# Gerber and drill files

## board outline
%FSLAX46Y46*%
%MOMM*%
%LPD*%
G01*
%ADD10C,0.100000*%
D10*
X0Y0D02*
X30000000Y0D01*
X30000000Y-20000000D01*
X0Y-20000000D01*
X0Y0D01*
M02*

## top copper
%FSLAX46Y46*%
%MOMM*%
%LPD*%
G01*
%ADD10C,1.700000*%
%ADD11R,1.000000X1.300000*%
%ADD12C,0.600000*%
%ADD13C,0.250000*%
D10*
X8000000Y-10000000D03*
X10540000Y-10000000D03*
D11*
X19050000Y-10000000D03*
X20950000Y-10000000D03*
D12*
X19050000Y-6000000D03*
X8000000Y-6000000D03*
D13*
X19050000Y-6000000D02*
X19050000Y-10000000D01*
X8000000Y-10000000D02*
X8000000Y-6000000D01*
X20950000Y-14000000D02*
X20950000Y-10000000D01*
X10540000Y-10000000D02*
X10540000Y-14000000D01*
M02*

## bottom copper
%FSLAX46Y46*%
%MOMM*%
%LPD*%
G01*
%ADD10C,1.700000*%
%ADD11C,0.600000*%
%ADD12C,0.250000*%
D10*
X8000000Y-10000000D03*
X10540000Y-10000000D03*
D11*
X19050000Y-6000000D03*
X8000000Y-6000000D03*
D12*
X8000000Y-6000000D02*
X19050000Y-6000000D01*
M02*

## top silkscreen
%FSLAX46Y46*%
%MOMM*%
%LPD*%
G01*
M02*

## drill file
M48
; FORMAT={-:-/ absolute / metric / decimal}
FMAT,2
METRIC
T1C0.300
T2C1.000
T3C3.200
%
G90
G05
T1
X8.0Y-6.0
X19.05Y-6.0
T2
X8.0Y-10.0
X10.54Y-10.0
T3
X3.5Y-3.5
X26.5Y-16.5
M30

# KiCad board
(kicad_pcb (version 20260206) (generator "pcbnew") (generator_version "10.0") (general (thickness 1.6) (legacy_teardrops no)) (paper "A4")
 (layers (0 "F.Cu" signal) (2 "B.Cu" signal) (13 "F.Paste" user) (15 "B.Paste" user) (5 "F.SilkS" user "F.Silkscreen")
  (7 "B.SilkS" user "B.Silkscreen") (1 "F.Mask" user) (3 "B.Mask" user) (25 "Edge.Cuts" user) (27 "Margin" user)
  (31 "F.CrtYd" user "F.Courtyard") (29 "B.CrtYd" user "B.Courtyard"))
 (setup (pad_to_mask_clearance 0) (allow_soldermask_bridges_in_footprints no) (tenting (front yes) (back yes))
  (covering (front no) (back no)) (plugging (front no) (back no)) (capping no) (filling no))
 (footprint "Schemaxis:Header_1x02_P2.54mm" (layer "F.Cu") (at 8 10 90)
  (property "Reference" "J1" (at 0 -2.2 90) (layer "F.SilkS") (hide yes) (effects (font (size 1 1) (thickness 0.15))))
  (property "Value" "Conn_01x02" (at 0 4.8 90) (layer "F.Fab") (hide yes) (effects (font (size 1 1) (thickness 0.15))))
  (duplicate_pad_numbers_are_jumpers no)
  (pad "1" thru_hole circle (at 0 0 90) (size 1.7 1.7) (drill 1) (layers "*.Cu" "*.Mask") (remove_unused_layers no) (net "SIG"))
  (pad "2" thru_hole circle (at 0 2.54 90) (size 1.7 1.7) (drill 1) (layers "*.Cu" "*.Mask") (remove_unused_layers no) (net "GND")))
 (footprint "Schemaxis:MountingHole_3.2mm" (layer "F.Cu") (at 3.5 3.5)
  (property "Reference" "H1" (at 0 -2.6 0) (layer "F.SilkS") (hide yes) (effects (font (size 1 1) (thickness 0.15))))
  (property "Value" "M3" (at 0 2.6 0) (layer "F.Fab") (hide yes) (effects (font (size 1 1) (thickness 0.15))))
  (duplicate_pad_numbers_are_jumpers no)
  (pad "" np_thru_hole circle (at 0 0) (size 3.2 3.2) (drill 3.2) (layers "*.Cu" "*.Mask")))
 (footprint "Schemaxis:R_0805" (layer "F.Cu") (at 20 10)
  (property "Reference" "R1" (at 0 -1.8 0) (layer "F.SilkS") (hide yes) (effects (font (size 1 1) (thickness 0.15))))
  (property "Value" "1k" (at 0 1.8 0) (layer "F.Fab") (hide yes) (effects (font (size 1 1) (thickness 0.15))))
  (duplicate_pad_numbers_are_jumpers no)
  (pad "1" smd rect (at -0.95 0) (size 1 1.3) (layers "F.Cu" "F.Mask" "F.Paste") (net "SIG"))
  (pad "2" smd rect (at 0.95 0) (size 1 1.3) (layers "F.Cu" "F.Mask" "F.Paste") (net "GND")))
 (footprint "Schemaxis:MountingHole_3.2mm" (layer "F.Cu") (at 26.5 16.5)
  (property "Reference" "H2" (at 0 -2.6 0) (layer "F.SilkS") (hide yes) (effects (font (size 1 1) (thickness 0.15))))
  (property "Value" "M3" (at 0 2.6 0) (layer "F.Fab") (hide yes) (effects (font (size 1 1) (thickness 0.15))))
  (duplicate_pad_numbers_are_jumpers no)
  (pad "" np_thru_hole circle (at 0 0) (size 3.2 3.2) (drill 3.2) (layers "*.Cu" "*.Mask")))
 (gr_rect (start 0 0) (end 30 20) (stroke (width 0.1) (type default)) (fill no) (layer "Edge.Cuts"))
 (segment (start 19.05 6) (end 19.05 10) (width 0.25) (layer "F.Cu") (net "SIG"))
 (segment (start 8 10) (end 8 6) (width 0.25) (layer "F.Cu") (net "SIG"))
 (via (at 19.05 6) (size 0.6) (drill 0.3) (layers "F.Cu" "B.Cu") (capping no) (covering (front no) (back no))
  (plugging (front no) (back no)) (filling no) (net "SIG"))
 (via (at 8 6) (size 0.6) (drill 0.3) (layers "F.Cu" "B.Cu") (capping no) (covering (front no) (back no)) (plugging (front no) (back no))
  (filling no) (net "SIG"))
 (segment (start 8 6) (end 19.05 6) (width 0.25) (layer "B.Cu") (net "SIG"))
 (segment (start 20.95 14) (end 20.95 10) (width 0.25) (layer "F.Cu") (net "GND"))
 (segment (start 10.54 10) (end 10.54 14) (width 0.25) (layer "F.Cu") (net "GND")))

